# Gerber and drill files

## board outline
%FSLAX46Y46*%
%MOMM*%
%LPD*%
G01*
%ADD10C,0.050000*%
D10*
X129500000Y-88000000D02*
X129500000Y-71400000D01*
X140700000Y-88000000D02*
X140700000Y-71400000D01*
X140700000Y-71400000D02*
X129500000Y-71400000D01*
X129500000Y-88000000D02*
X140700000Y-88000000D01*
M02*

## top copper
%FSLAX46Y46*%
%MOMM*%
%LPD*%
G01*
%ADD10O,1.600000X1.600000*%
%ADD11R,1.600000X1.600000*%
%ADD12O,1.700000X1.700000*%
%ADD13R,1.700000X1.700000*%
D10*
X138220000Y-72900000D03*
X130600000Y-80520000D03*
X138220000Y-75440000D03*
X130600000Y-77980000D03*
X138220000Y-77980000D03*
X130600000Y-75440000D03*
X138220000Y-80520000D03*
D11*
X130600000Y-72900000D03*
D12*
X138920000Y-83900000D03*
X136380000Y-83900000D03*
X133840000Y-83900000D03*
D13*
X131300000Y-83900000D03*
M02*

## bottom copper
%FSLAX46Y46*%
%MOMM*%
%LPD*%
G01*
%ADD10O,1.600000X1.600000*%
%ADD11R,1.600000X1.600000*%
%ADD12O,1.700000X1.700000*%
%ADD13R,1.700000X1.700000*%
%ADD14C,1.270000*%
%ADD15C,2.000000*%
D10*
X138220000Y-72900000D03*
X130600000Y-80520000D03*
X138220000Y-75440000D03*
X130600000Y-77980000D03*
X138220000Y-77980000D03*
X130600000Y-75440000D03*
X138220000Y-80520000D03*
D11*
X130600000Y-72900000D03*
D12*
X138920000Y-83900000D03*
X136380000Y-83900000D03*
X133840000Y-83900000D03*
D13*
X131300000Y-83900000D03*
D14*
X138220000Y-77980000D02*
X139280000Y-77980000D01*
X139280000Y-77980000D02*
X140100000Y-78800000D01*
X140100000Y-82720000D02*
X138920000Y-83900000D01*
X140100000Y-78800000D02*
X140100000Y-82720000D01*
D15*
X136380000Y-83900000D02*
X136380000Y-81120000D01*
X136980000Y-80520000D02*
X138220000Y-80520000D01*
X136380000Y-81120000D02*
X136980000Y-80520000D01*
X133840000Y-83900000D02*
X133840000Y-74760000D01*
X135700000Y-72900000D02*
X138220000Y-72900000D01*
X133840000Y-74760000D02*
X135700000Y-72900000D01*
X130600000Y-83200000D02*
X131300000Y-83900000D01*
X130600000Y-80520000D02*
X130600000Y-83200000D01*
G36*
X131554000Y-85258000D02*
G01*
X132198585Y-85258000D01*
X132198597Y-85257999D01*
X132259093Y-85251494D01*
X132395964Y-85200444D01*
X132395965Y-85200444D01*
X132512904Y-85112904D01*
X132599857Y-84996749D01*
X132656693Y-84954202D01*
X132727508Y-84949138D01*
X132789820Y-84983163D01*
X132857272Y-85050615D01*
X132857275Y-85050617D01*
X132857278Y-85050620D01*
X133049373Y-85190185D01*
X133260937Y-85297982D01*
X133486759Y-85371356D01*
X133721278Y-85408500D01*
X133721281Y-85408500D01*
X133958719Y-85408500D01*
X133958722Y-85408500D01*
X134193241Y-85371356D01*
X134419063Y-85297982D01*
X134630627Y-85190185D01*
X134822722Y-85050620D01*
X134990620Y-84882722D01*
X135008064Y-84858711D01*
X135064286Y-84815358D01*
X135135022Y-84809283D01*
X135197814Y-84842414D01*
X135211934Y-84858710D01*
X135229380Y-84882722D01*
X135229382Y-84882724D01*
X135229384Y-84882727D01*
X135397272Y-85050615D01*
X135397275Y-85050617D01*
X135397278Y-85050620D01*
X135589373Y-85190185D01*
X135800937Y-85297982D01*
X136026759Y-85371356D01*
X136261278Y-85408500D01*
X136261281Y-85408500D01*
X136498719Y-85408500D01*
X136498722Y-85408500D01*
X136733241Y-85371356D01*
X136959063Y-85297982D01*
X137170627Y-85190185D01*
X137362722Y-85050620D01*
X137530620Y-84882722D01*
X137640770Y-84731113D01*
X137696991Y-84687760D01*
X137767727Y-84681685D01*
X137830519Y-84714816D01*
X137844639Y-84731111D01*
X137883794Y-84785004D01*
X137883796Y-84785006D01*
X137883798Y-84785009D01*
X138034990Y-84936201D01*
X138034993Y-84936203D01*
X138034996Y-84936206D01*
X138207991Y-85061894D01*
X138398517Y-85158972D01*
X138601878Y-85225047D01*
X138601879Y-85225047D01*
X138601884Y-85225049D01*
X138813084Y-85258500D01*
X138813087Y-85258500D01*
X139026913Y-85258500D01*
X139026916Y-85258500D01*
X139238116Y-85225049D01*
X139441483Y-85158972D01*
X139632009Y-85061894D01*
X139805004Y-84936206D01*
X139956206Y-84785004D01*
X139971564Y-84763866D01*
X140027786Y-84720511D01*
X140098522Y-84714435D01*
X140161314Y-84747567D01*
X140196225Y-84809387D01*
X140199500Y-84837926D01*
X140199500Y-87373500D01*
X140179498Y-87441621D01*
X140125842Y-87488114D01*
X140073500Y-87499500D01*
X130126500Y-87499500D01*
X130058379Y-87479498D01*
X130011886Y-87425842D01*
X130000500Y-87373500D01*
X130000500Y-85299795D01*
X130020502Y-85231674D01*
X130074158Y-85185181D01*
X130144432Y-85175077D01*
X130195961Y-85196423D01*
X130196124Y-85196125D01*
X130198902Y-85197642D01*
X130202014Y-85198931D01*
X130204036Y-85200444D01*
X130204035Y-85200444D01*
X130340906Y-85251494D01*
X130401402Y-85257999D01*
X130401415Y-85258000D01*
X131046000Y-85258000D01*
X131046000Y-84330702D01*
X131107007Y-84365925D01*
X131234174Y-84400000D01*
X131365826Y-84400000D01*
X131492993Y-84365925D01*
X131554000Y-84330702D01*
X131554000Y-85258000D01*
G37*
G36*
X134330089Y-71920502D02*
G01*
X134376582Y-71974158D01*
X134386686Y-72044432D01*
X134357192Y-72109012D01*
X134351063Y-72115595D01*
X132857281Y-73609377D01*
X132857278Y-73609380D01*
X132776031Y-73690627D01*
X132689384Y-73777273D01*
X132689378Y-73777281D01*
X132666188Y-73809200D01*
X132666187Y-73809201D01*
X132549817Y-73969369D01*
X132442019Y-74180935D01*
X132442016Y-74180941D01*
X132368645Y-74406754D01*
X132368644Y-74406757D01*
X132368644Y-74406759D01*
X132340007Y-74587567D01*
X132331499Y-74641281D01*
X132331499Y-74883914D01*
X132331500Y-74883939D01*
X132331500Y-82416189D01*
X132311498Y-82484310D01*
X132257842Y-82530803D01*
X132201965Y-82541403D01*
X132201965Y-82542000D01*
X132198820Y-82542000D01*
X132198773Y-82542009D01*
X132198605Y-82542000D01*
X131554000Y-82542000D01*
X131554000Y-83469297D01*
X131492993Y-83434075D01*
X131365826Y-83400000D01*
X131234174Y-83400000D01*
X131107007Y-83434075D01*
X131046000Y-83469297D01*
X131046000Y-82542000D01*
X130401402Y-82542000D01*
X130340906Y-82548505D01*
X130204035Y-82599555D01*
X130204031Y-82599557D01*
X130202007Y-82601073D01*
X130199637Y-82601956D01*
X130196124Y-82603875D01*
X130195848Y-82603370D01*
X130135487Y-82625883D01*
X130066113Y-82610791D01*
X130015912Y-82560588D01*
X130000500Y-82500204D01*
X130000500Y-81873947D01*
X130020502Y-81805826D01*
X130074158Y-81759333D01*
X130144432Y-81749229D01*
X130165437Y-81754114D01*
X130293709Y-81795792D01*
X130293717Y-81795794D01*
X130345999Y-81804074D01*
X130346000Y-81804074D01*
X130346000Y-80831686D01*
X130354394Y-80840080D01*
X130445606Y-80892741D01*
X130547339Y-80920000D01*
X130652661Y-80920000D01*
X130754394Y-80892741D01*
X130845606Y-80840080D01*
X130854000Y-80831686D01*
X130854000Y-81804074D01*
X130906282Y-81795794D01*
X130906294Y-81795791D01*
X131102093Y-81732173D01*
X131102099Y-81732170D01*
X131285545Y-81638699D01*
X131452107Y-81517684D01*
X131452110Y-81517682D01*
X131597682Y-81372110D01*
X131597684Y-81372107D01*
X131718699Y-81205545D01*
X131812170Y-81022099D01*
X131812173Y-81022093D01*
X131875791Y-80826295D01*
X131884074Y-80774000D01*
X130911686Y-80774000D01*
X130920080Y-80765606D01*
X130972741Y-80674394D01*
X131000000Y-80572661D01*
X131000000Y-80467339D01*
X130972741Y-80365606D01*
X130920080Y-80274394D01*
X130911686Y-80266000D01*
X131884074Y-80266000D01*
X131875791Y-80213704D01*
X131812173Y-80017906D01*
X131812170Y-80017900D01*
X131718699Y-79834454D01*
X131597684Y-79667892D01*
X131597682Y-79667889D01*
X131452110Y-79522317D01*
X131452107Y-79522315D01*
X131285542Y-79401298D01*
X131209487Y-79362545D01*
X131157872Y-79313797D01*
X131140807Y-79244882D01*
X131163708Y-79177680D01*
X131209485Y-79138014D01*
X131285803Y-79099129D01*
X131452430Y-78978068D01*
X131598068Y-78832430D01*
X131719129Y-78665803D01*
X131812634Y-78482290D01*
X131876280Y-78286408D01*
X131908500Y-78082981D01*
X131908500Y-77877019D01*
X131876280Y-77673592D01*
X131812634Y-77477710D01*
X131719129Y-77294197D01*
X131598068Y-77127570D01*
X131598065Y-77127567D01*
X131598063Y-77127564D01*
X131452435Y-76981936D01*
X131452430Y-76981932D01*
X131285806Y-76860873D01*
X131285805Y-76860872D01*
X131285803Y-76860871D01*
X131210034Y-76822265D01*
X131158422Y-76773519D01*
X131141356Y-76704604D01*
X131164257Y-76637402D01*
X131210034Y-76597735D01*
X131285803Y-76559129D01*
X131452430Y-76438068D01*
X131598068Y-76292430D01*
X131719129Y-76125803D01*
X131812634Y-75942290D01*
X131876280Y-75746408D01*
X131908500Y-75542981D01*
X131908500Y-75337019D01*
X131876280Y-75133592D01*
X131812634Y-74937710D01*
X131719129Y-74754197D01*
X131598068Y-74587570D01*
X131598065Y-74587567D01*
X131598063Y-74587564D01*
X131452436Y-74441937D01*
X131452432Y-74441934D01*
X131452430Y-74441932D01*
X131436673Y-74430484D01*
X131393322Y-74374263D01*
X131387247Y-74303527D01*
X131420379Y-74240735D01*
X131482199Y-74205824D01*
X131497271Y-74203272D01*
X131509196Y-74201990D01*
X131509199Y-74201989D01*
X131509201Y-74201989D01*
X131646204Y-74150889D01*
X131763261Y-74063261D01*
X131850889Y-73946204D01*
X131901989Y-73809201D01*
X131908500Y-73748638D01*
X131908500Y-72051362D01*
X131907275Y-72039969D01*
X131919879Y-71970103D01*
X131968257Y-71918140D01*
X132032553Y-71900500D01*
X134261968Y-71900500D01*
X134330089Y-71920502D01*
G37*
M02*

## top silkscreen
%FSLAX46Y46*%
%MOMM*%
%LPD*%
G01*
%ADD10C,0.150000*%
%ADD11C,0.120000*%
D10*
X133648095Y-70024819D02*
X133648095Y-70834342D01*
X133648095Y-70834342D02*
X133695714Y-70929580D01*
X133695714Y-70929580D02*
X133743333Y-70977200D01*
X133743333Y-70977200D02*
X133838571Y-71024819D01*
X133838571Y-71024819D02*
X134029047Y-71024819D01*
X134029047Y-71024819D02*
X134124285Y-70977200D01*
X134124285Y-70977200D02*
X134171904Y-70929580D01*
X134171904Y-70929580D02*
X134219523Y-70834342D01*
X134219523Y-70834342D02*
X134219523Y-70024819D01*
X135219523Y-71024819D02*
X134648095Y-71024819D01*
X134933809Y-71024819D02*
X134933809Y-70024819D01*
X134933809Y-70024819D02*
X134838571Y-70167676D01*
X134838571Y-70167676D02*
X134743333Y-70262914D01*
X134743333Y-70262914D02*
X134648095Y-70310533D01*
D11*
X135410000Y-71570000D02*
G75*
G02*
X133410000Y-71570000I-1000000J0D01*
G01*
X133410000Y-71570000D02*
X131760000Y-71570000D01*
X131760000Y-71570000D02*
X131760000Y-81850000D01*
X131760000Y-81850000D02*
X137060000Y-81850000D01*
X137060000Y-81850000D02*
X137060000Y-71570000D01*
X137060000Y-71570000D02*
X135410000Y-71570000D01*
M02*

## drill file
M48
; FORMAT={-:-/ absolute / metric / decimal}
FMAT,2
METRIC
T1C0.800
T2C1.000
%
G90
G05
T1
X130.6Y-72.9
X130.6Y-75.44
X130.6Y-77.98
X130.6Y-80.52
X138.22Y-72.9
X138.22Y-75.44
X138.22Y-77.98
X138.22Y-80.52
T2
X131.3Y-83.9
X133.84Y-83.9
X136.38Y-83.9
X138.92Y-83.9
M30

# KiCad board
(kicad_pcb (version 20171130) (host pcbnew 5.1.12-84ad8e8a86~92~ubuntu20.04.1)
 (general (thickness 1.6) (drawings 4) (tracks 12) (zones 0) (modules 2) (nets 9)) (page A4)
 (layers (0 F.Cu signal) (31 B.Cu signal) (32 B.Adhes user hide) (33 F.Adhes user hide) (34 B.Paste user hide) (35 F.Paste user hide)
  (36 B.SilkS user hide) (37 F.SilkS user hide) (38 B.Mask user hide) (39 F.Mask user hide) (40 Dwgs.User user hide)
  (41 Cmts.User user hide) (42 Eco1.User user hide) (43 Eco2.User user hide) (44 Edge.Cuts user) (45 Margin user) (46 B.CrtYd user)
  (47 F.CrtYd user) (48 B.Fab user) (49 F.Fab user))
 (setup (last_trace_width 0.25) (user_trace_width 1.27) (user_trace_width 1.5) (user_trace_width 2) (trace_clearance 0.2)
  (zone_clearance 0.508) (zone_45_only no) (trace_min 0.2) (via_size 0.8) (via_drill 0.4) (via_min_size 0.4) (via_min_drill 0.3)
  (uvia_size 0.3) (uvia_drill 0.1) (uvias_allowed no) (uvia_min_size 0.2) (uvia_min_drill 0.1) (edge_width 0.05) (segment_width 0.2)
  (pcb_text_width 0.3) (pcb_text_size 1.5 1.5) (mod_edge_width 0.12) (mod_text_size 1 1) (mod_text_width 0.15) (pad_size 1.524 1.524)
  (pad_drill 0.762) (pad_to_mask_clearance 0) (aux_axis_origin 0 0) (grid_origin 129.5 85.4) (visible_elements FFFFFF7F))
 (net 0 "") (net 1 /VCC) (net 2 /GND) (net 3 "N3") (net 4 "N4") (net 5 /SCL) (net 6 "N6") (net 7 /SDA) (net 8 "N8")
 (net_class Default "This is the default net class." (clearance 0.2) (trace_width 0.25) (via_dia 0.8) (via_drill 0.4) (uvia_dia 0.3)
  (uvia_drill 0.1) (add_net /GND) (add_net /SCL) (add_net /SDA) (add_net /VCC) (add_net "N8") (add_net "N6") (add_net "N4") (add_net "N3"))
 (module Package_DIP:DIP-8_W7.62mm (layer F.Cu) (at 130.6 72.9)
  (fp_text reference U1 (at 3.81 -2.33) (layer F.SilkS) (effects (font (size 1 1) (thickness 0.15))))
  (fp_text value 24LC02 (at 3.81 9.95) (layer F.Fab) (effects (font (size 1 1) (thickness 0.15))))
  (fp_arc (start 3.81 -1.33) (end 2.81 -1.33) (angle -180) (layer F.SilkS) (width 0.12))
  (fp_line (start 2.81 -1.33) (end 1.16 -1.33) (layer F.SilkS) (width 0.12))
  (fp_line (start 1.16 -1.33) (end 1.16 8.95) (layer F.SilkS) (width 0.12))
  (fp_line (start 1.16 8.95) (end 6.46 8.95) (layer F.SilkS) (width 0.12))
  (fp_line (start 6.46 8.95) (end 6.46 -1.33) (layer F.SilkS) (width 0.12))
  (fp_line (start 6.46 -1.33) (end 4.81 -1.33) (layer F.SilkS) (width 0.12))
  (pad 8 thru_hole oval (at 7.62 0) (size 1.6 1.6) (drill 0.8) (layers *.Cu *.Mask) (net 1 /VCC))
  (pad 4 thru_hole oval (at 0 7.62) (size 1.6 1.6) (drill 0.8) (layers *.Cu *.Mask) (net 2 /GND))
  (pad 7 thru_hole oval (at 7.62 2.54) (size 1.6 1.6) (drill 0.8) (layers *.Cu *.Mask) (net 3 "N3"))
  (pad 3 thru_hole oval (at 0 5.08) (size 1.6 1.6) (drill 0.8) (layers *.Cu *.Mask) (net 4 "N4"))
  (pad 6 thru_hole oval (at 7.62 5.08) (size 1.6 1.6) (drill 0.8) (layers *.Cu *.Mask) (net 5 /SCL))
  (pad 2 thru_hole oval (at 0 2.54) (size 1.6 1.6) (drill 0.8) (layers *.Cu *.Mask) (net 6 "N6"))
  (pad 5 thru_hole oval (at 7.62 7.62) (size 1.6 1.6) (drill 0.8) (layers *.Cu *.Mask) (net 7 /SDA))
  (pad 1 thru_hole rect (at 0 0) (size 1.6 1.6) (drill 0.8) (layers *.Cu *.Mask) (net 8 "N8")))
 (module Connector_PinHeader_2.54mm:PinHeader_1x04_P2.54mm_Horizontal (layer B.Cu) (at 131.3 83.9 270)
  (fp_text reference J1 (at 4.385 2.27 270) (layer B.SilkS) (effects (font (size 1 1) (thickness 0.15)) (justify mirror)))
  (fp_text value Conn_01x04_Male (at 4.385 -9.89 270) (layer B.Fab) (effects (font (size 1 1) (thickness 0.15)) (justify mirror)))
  (pad 4 thru_hole oval (at 0 -7.62 270) (size 1.7 1.7) (drill 1) (layers *.Cu *.Mask) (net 5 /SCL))
  (pad 3 thru_hole oval (at 0 -5.08 270) (size 1.7 1.7) (drill 1) (layers *.Cu *.Mask) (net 7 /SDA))
  (pad 2 thru_hole oval (at 0 -2.54 270) (size 1.7 1.7) (drill 1) (layers *.Cu *.Mask) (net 1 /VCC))
  (pad 1 thru_hole rect (at 0 0 270) (size 1.7 1.7) (drill 1) (layers *.Cu *.Mask) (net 2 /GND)))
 (gr_line (start 129.5 88) (end 129.5 71.4) (layer Edge.Cuts) (width 0.05))
 (gr_line (start 140.7 88) (end 140.7 71.4) (layer Edge.Cuts) (width 0.05))
 (gr_line (start 140.7 71.4) (end 129.5 71.4) (layer Edge.Cuts) (width 0.05))
 (gr_line (start 129.5 88) (end 140.7 88) (layer Edge.Cuts) (width 0.05))
 (segment (start 138.22 77.98) (end 139.28 77.98) (width 1.27) (layer B.Cu) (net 5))
 (segment (start 139.28 77.98) (end 140.1 78.8) (width 1.27) (layer B.Cu) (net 5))
 (segment (start 140.1 82.72) (end 138.92 83.9) (width 1.27) (layer B.Cu) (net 5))
 (segment (start 140.1 78.8) (end 140.1 82.72) (width 1.27) (layer B.Cu) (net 5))
 (segment (start 136.38 83.9) (end 136.38 81.12) (width 2) (layer B.Cu) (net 7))
 (segment (start 136.98 80.52) (end 138.22 80.52) (width 2) (layer B.Cu) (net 7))
 (segment (start 136.38 81.12) (end 136.98 80.52) (width 2) (layer B.Cu) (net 7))
 (segment (start 133.84 83.9) (end 133.84 74.76) (width 2) (layer B.Cu) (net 1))
 (segment (start 135.7 72.9) (end 138.22 72.9) (width 2) (layer B.Cu) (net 1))
 (segment (start 133.84 74.76) (end 135.7 72.9) (width 2) (layer B.Cu) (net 1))
 (segment (start 130.6 83.2) (end 131.3 83.9) (width 2) (layer B.Cu) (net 2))
 (segment (start 130.6 80.52) (end 130.6 83.2) (width 2) (layer B.Cu) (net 2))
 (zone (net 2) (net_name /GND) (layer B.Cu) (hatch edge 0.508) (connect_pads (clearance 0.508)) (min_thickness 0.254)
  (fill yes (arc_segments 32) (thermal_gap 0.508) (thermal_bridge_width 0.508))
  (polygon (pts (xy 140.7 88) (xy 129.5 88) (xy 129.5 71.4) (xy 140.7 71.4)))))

